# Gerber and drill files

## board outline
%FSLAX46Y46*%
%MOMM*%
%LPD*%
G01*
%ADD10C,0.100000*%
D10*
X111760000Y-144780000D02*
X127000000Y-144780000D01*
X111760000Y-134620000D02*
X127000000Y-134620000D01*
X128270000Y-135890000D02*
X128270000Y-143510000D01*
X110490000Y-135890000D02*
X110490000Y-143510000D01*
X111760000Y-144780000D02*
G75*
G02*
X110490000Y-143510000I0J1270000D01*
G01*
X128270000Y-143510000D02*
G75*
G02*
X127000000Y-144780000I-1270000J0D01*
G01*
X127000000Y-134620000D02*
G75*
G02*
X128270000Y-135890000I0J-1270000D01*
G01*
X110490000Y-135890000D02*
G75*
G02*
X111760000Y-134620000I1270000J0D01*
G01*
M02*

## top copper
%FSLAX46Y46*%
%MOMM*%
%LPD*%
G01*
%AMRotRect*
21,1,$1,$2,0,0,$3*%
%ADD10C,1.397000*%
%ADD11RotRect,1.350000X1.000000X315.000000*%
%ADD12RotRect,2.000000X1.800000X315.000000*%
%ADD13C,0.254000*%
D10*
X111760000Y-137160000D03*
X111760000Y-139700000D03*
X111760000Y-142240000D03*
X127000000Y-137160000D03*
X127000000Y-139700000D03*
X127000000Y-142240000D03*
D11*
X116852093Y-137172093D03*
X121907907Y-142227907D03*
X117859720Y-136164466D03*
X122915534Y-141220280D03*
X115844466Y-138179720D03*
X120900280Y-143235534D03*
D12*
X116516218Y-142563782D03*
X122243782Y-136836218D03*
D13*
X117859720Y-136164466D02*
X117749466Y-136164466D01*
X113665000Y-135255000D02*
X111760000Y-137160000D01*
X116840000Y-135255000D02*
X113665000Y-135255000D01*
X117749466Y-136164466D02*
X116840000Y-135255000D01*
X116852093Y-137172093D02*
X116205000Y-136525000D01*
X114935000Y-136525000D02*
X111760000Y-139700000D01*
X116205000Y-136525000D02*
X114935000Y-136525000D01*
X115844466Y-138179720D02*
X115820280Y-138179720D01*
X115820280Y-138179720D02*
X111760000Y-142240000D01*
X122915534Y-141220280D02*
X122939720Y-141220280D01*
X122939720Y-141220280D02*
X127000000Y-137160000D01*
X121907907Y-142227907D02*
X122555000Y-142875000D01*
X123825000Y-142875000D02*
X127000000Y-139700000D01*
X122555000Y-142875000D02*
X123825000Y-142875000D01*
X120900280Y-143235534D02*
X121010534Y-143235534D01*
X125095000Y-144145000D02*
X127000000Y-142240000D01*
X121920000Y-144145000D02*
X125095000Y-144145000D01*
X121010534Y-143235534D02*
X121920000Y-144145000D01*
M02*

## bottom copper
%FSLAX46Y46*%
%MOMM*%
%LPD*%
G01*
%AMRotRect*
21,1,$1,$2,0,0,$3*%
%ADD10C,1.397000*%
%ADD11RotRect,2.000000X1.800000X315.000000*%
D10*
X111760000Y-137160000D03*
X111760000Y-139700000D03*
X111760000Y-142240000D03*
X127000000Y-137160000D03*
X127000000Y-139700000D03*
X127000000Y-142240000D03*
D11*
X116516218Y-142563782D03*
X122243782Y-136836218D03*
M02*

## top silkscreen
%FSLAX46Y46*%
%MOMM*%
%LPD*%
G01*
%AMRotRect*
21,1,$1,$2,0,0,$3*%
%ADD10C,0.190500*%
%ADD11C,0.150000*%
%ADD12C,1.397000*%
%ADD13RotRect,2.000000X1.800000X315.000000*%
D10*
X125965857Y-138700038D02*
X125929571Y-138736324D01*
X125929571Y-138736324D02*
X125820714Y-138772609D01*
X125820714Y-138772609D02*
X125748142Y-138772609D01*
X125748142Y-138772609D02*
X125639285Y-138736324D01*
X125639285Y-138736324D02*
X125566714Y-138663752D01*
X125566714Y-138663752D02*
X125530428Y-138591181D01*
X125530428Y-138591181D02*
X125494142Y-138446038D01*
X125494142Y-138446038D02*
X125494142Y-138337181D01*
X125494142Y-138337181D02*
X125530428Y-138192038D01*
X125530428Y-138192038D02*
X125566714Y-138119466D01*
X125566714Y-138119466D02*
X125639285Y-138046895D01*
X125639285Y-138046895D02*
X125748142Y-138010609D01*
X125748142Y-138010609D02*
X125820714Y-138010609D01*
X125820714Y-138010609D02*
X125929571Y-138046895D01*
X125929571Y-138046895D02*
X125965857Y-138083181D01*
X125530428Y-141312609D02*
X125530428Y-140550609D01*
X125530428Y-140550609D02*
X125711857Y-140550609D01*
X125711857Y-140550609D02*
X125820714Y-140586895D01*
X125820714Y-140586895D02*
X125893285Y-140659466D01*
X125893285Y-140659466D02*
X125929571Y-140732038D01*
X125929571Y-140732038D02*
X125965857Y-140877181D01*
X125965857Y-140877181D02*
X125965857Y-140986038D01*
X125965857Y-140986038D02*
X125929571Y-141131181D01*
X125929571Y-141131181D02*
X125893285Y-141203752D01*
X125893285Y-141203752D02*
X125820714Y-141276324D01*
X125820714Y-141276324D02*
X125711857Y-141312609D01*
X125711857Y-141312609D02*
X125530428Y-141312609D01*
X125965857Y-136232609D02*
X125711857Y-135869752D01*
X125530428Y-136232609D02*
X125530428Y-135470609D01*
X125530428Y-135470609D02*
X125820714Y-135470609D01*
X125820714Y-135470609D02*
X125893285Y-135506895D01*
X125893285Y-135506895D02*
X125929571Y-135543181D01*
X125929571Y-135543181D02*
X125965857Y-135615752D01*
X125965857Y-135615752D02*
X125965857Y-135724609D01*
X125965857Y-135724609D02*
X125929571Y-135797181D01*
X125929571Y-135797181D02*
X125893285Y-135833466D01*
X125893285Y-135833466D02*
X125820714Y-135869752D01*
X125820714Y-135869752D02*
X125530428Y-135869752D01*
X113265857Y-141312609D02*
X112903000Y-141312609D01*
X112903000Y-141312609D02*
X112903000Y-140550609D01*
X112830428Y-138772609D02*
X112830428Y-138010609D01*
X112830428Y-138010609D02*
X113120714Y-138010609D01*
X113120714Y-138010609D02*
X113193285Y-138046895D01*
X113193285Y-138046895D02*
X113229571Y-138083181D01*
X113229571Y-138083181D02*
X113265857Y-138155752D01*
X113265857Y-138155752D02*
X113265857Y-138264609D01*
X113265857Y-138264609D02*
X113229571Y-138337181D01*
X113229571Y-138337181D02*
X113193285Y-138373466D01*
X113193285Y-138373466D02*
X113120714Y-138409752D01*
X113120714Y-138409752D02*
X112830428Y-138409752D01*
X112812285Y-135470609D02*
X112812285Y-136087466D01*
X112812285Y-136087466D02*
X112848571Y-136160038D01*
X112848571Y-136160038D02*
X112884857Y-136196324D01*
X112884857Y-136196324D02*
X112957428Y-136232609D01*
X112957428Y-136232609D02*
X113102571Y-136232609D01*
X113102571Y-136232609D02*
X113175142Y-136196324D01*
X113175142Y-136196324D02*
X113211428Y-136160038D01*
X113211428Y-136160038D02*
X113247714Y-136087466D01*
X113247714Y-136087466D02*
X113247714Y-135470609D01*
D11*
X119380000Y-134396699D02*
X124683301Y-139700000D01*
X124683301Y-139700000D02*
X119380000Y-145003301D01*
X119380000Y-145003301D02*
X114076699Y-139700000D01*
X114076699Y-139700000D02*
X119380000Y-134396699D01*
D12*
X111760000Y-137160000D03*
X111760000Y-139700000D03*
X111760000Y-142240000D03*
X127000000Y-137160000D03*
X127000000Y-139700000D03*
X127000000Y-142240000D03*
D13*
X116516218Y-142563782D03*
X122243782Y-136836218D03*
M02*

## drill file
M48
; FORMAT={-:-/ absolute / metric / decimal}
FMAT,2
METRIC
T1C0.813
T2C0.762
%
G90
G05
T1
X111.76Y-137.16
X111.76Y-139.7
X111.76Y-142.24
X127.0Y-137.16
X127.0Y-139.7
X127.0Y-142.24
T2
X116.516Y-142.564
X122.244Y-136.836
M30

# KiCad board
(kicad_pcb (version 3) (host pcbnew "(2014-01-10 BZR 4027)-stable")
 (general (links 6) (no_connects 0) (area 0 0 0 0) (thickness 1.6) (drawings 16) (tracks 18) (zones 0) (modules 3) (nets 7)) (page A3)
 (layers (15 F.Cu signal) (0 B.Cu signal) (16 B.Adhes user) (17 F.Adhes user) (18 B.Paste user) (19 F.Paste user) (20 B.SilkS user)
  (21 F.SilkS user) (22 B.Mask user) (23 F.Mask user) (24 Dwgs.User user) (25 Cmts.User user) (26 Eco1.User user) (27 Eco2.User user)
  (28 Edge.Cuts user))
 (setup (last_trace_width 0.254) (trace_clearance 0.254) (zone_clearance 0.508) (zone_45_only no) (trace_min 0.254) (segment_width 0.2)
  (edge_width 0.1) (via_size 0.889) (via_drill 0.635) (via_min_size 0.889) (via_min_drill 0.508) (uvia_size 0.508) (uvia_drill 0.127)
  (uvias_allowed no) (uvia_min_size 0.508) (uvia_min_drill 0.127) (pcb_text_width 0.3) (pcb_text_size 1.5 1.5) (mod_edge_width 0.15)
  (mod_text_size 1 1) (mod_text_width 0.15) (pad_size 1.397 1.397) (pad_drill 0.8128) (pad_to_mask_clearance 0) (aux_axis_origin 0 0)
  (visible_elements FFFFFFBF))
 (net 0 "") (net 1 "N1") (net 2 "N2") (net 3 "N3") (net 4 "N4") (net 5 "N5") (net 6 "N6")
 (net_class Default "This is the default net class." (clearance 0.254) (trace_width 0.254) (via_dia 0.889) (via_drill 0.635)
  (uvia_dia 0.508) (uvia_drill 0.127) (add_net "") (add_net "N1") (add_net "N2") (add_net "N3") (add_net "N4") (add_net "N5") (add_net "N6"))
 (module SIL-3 (layer F.Cu) (at 111.76 139.7 270)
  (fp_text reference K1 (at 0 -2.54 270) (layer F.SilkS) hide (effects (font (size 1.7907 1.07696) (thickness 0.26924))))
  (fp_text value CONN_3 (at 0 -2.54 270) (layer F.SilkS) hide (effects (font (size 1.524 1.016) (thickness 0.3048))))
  (pad 1 thru_hole circle (at -2.54 0 270) (size 1.397 1.397) (drill 0.8128) (layers *.Cu *.Mask F.SilkS) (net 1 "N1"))
  (pad 2 thru_hole circle (at 0 0 270) (size 1.397 1.397) (drill 0.8128) (layers *.Cu *.Mask F.SilkS) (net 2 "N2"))
  (pad 3 thru_hole circle (at 2.54 0 270) (size 1.397 1.397) (drill 0.8128) (layers *.Cu *.Mask F.SilkS) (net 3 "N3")))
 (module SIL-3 (layer F.Cu) (at 127 139.7 270)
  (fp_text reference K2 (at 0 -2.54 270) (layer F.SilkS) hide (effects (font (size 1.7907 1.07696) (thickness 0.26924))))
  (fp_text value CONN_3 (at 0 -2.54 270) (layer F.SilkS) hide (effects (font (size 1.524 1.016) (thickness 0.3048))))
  (pad 1 thru_hole circle (at -2.54 0 270) (size 1.397 1.397) (drill 0.8128) (layers *.Cu *.Mask F.SilkS) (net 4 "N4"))
  (pad 2 thru_hole circle (at 0 0 270) (size 1.397 1.397) (drill 0.8128) (layers *.Cu *.Mask F.SilkS) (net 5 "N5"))
  (pad 3 thru_hole circle (at 2.54 0 270) (size 1.397 1.397) (drill 0.8128) (layers *.Cu *.Mask F.SilkS) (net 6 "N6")))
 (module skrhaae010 (layer F.Cu) (at 119.38 139.7 315)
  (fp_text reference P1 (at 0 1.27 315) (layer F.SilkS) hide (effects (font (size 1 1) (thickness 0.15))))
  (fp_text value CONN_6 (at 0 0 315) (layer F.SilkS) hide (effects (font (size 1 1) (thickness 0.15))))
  (fp_line (start -3.75 -3.75) (end 3.75 -3.75) (layer F.SilkS) (width 0.15))
  (fp_line (start 3.75 -3.75) (end 3.75 3.75) (layer F.SilkS) (width 0.15))
  (fp_line (start 3.75 3.75) (end -3.75 3.75) (layer F.SilkS) (width 0.15))
  (fp_line (start -3.75 3.75) (end -3.75 -3.75) (layer F.SilkS) (width 0.15))
  (pad 2 smd rect (at -3.575 0 315) (size 1.35 1) (layers F.Cu F.Paste F.Mask) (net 2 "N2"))
  (pad 5 smd rect (at 3.575 0 315) (size 1.35 1) (layers F.Cu F.Paste F.Mask) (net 5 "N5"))
  (pad 1 smd rect (at -3.575 -1.425 315) (size 1.35 1) (layers F.Cu F.Paste F.Mask) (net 1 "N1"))
  (pad 4 smd rect (at 3.575 -1.425 315) (size 1.35 1) (layers F.Cu F.Paste F.Mask) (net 4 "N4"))
  (pad 3 smd rect (at -3.575 1.425 315) (size 1.35 1) (layers F.Cu F.Paste F.Mask) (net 3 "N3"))
  (pad 6 smd rect (at 3.575 1.425 315) (size 1.35 1) (layers F.Cu F.Paste F.Mask) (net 6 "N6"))
  (pad "" np_thru_hole rect (at 0 4.05 315) (size 2 1.8) (layers *.Cu *.Mask F.SilkS))
  (pad "" np_thru_hole rect (at 0 -4.05 315) (size 2 1.8) (layers *.Cu *.Mask F.SilkS)))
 (gr_line (start 111.76 144.78) (end 127 144.78) (angle 90) (layer Edge.Cuts) (width 0.1))
 (gr_line (start 111.76 134.62) (end 127 134.62) (angle 90) (layer Edge.Cuts) (width 0.1))
 (gr_line (start 128.27 135.89) (end 128.27 143.51) (angle 90) (layer Edge.Cuts) (width 0.1))
 (gr_line (start 110.49 135.89) (end 110.49 143.51) (angle 90) (layer Edge.Cuts) (width 0.1))
 (gr_arc (start 111.76 143.51) (end 111.76 144.78) (angle 90) (layer Edge.Cuts) (width 0.1))
 (gr_arc (start 127 143.51) (end 128.27 143.51) (angle 90) (layer Edge.Cuts) (width 0.1))
 (gr_arc (start 127 135.89) (end 127 134.62) (angle 90) (layer Edge.Cuts) (width 0.1))
 (gr_arc (start 111.76 135.89) (end 110.49 135.89) (angle 90) (layer Edge.Cuts) (width 0.1))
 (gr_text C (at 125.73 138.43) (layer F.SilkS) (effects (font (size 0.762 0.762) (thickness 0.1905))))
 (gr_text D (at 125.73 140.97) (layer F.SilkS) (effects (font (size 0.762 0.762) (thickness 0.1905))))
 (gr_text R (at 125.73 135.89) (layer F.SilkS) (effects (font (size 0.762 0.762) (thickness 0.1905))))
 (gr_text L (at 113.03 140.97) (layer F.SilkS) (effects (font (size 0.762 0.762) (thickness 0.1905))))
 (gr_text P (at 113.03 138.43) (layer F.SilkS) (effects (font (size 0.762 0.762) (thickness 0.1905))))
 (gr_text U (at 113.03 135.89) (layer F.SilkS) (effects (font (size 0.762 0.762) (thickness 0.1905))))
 (segment (start 117.85972 136.164466) (end 117.749466 136.164466) (width 0.254) (layer F.Cu) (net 1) (status C00000))
 (segment (start 113.665 135.255) (end 111.76 137.16) (width 0.254) (layer F.Cu) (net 1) (status 800000))
 (segment (start 116.84 135.255) (end 113.665 135.255) (width 0.254) (layer F.Cu) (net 1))
 (segment (start 117.749466 136.164466) (end 116.84 135.255) (width 0.254) (layer F.Cu) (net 1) (status 400000))
 (segment (start 116.852093 137.172093) (end 116.205 136.525) (width 0.254) (layer F.Cu) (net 2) (status 400000))
 (segment (start 114.935 136.525) (end 111.76 139.7) (width 0.254) (layer F.Cu) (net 2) (status 800000))
 (segment (start 116.205 136.525) (end 114.935 136.525) (width 0.254) (layer F.Cu) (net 2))
 (segment (start 115.844466 138.17972) (end 115.82028 138.17972) (width 0.254) (layer F.Cu) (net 3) (status C00000))
 (segment (start 115.82028 138.17972) (end 111.76 142.24) (width 0.254) (layer F.Cu) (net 3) (status C00000))
 (segment (start 122.915534 141.22028) (end 122.93972 141.22028) (width 0.254) (layer F.Cu) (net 4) (status C00000))
 (segment (start 122.93972 141.22028) (end 127 137.16) (width 0.254) (layer F.Cu) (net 4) (status C00000))
 (segment (start 121.907907 142.227907) (end 122.555 142.875) (width 0.254) (layer F.Cu) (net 5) (status 400000))
 (segment (start 123.825 142.875) (end 127 139.7) (width 0.254) (layer F.Cu) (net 5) (status 800000))
 (segment (start 122.555 142.875) (end 123.825 142.875) (width 0.254) (layer F.Cu) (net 5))
 (segment (start 120.90028 143.235534) (end 121.010534 143.235534) (width 0.254) (layer F.Cu) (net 6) (status C00000))
 (segment (start 125.095 144.145) (end 127 142.24) (width 0.254) (layer F.Cu) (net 6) (status 800000))
 (segment (start 121.92 144.145) (end 125.095 144.145) (width 0.254) (layer F.Cu) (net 6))
 (segment (start 121.010534 143.235534) (end 121.92 144.145) (width 0.254) (layer F.Cu) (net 6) (status 400000)))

